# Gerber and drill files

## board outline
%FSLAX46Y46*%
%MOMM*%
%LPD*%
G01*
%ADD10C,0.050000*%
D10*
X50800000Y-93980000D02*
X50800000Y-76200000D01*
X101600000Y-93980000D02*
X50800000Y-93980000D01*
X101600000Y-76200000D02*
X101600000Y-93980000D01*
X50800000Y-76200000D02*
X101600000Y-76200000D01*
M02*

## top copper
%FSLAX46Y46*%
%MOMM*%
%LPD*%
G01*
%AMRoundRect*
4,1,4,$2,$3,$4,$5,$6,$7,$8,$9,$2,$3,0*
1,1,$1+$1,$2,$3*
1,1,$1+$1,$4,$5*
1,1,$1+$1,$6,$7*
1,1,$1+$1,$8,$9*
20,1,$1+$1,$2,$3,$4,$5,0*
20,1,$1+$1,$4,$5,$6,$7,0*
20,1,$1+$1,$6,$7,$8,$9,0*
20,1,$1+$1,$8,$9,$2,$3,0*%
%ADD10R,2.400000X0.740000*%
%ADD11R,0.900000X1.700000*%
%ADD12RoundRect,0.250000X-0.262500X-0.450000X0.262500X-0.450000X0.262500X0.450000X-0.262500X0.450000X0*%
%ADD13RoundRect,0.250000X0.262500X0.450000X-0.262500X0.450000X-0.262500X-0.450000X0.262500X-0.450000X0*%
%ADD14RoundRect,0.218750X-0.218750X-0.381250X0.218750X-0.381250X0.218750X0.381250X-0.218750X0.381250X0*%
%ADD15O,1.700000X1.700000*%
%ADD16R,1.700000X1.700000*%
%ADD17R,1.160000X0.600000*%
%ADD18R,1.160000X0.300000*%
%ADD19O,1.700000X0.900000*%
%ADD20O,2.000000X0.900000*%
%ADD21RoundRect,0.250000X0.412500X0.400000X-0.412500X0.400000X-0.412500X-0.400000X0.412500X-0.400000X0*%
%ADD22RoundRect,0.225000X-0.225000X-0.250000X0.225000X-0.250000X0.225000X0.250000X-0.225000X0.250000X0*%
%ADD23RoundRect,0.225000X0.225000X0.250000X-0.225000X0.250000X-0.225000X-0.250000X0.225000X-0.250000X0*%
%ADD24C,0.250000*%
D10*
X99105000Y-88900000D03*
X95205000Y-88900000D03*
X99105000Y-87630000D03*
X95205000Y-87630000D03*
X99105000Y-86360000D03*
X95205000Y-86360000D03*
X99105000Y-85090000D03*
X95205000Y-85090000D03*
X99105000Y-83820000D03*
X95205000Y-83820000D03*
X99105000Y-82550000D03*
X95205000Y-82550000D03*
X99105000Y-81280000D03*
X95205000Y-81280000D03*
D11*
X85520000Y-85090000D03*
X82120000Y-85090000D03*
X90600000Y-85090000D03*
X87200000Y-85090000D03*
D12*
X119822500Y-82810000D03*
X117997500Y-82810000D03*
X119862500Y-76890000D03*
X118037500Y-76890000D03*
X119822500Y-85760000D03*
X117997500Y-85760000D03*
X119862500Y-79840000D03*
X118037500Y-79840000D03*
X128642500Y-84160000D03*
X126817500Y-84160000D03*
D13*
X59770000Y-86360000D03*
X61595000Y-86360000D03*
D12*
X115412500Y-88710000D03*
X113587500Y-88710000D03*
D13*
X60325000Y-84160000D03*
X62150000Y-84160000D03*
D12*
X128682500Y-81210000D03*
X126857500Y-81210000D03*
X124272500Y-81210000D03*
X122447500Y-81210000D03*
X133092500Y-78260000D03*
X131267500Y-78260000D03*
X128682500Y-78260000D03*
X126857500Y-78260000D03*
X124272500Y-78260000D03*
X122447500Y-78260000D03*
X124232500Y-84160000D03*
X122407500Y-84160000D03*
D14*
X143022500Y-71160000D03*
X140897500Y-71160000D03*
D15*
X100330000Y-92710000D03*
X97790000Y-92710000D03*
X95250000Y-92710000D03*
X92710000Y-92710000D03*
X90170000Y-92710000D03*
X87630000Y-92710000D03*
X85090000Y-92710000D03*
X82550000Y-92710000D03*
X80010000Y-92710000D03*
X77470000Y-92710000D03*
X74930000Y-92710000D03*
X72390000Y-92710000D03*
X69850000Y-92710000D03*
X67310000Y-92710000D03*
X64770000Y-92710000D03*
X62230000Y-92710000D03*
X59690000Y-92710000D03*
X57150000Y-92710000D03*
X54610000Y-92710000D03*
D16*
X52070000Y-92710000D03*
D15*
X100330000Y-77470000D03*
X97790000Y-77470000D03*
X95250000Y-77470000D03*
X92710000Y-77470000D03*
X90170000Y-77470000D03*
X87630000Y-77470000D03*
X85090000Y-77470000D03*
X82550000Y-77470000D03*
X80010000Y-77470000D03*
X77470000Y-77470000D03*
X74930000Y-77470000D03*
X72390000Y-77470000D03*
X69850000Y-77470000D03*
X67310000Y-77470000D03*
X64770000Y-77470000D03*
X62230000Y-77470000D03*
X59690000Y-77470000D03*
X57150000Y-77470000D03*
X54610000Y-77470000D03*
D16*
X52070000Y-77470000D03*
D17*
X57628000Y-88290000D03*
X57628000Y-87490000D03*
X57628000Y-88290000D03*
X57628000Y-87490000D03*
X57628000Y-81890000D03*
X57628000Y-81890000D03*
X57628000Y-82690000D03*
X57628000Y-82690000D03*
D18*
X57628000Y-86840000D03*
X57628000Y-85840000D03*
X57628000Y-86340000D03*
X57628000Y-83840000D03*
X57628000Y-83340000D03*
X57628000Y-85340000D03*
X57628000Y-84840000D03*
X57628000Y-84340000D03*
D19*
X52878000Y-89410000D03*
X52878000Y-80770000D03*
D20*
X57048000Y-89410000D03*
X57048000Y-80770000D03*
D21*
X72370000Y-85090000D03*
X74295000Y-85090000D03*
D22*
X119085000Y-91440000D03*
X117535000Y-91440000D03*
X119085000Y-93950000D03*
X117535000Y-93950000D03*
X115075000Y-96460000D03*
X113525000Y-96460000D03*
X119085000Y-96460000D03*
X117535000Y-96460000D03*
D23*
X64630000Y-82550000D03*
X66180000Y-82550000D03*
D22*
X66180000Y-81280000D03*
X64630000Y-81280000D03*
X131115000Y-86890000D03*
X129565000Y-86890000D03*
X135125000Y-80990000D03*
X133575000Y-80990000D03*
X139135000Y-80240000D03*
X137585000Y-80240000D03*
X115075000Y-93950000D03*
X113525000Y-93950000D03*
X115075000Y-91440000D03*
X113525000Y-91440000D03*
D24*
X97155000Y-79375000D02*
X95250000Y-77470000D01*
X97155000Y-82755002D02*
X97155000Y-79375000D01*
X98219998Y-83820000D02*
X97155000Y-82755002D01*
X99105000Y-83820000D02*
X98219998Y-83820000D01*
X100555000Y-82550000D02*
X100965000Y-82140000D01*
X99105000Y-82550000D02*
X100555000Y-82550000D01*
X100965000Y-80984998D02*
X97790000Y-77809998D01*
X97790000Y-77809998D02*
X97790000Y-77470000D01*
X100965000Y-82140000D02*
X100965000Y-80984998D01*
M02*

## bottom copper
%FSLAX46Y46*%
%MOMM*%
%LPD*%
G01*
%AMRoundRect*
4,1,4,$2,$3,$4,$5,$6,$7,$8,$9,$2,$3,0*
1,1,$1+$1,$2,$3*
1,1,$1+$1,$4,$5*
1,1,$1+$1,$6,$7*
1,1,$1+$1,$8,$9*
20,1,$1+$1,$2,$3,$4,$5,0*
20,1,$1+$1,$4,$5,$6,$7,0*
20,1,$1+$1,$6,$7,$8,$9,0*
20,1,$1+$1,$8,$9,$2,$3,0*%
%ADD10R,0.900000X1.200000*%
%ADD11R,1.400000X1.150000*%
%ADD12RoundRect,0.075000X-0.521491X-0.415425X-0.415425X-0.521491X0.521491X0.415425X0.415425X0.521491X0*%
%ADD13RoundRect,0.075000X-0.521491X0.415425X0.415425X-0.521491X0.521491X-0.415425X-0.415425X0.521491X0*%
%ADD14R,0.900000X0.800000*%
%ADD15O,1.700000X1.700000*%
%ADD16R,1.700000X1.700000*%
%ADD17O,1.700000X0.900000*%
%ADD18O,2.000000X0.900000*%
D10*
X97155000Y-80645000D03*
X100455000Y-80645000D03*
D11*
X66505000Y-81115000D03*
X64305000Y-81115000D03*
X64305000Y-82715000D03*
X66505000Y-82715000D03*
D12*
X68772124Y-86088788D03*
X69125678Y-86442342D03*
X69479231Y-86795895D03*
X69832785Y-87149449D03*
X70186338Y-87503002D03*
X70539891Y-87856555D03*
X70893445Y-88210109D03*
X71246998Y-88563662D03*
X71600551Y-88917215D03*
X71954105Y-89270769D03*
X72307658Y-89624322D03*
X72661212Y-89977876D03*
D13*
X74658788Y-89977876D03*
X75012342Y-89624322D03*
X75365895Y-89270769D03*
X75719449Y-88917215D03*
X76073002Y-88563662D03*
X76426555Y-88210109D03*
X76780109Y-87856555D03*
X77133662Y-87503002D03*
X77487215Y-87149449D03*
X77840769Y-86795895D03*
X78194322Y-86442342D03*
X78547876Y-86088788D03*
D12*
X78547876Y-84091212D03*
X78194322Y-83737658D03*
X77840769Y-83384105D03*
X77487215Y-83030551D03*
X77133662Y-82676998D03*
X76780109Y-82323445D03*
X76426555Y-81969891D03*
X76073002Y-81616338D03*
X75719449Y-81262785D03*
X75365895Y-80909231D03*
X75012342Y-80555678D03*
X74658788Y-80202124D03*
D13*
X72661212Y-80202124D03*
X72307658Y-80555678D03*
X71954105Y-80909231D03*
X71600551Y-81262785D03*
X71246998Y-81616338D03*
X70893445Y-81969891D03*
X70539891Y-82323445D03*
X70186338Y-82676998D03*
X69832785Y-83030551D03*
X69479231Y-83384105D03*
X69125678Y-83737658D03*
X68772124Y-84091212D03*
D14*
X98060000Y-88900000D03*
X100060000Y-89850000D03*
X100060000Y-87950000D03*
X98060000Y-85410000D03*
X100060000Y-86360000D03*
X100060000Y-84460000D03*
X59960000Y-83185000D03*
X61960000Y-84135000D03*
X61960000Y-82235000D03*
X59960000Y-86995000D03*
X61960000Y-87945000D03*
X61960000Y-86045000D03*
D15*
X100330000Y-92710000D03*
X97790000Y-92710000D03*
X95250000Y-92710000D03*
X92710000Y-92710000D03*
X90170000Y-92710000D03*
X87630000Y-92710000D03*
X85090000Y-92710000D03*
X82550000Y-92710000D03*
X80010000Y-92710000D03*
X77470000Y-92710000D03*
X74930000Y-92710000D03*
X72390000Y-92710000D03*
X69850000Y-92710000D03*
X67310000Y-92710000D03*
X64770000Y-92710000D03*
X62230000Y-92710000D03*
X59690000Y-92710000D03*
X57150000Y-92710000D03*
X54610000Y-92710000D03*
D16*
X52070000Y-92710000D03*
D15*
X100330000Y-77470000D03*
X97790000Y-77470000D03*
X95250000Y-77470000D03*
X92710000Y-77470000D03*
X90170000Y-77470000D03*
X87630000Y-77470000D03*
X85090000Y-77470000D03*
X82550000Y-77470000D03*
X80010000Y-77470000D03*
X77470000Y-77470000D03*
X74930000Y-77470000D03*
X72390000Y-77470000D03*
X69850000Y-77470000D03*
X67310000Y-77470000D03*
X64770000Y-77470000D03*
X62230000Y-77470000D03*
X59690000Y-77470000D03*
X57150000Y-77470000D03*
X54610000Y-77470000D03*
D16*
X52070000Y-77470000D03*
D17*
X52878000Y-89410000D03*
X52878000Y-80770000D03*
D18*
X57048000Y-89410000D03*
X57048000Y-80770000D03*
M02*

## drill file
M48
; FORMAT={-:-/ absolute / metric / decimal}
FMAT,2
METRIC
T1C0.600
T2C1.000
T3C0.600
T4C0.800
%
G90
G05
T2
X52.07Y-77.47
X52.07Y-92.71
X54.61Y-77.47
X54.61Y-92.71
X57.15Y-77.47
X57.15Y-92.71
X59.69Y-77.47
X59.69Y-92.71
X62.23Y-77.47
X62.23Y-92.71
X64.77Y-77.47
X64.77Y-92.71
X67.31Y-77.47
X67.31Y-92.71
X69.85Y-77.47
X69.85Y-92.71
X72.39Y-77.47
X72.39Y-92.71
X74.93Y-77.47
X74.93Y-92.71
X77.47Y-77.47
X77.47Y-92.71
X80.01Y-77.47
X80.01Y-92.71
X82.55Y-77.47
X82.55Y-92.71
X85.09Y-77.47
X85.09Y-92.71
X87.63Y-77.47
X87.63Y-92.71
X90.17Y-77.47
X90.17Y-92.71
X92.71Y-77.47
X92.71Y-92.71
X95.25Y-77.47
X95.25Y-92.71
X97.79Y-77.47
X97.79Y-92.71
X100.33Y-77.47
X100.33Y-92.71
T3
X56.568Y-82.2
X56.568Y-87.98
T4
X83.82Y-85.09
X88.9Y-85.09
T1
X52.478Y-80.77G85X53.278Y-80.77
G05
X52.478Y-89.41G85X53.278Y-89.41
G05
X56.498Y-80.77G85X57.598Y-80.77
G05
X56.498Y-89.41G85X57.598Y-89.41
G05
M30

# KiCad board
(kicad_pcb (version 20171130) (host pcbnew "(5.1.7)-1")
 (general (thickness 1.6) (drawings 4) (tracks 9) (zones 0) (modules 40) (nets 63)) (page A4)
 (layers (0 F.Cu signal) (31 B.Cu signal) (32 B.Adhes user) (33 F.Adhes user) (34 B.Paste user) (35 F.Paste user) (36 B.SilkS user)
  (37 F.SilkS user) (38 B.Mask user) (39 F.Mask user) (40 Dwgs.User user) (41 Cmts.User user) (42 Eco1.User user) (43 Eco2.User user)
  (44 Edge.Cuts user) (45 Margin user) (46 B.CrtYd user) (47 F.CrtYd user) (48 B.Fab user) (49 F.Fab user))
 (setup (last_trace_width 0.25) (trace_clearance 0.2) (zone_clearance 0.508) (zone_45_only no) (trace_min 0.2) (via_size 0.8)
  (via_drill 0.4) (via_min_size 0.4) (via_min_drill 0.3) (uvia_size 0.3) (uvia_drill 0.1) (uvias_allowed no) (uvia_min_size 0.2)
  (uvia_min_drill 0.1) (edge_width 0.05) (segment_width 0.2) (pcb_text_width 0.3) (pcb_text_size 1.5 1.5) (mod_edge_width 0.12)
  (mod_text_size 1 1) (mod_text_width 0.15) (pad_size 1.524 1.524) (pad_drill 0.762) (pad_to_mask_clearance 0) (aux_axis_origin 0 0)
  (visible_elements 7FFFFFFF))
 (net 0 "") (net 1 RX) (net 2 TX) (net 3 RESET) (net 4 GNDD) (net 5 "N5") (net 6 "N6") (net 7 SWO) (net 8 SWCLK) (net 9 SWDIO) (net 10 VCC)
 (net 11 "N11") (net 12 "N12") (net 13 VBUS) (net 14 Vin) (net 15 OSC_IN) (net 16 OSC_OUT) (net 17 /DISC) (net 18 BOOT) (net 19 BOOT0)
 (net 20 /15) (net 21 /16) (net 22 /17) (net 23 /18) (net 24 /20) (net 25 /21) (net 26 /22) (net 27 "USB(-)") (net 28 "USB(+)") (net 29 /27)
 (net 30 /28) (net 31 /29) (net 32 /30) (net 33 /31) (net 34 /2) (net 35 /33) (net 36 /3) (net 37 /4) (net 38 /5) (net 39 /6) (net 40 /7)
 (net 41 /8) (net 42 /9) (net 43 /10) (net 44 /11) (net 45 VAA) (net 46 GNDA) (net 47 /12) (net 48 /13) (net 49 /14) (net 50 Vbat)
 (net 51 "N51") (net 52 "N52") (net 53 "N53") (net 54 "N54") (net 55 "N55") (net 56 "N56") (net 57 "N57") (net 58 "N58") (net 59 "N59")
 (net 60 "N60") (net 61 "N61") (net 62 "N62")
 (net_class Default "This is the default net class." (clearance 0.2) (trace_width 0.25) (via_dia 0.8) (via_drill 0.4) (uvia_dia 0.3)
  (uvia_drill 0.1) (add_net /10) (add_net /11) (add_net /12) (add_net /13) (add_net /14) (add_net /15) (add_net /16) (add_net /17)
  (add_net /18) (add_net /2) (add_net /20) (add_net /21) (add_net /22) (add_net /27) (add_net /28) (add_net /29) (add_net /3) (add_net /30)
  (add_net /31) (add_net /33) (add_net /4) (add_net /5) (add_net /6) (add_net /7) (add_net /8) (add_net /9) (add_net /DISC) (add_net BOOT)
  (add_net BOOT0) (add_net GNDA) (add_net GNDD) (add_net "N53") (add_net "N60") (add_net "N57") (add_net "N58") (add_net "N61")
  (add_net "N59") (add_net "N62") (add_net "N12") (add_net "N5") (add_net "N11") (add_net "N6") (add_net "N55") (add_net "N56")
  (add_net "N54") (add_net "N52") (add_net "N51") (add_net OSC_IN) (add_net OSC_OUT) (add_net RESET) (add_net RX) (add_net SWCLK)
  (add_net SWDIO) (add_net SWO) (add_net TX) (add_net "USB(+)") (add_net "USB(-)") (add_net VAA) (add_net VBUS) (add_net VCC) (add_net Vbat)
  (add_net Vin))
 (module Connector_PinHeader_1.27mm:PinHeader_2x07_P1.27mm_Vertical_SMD (layer F.Cu) (at 97.155 85.09)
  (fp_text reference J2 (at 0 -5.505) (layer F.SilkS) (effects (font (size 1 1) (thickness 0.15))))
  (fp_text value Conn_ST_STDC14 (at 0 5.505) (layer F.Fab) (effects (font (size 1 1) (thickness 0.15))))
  (pad 14 smd rect (at 1.95 3.81) (size 2.4 0.74) (layers F.Cu F.Paste F.Mask) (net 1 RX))
  (pad 13 smd rect (at -1.95 3.81) (size 2.4 0.74) (layers F.Cu F.Paste F.Mask) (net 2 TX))
  (pad 12 smd rect (at 1.95 2.54) (size 2.4 0.74) (layers F.Cu F.Paste F.Mask) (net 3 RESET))
  (pad 11 smd rect (at -1.95 2.54) (size 2.4 0.74) (layers F.Cu F.Paste F.Mask) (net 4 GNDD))
  (pad 10 smd rect (at 1.95 1.27) (size 2.4 0.74) (layers F.Cu F.Paste F.Mask) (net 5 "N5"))
  (pad 9 smd rect (at -1.95 1.27) (size 2.4 0.74) (layers F.Cu F.Paste F.Mask) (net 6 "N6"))
  (pad 8 smd rect (at 1.95 0) (size 2.4 0.74) (layers F.Cu F.Paste F.Mask) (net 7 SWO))
  (pad 7 smd rect (at -1.95 0) (size 2.4 0.74) (layers F.Cu F.Paste F.Mask) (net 4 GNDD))
  (pad 6 smd rect (at 1.95 -1.27) (size 2.4 0.74) (layers F.Cu F.Paste F.Mask) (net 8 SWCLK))
  (pad 5 smd rect (at -1.95 -1.27) (size 2.4 0.74) (layers F.Cu F.Paste F.Mask) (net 4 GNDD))
  (pad 4 smd rect (at 1.95 -2.54) (size 2.4 0.74) (layers F.Cu F.Paste F.Mask) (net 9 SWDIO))
  (pad 3 smd rect (at -1.95 -2.54) (size 2.4 0.74) (layers F.Cu F.Paste F.Mask) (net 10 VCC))
  (pad 2 smd rect (at 1.95 -3.81) (size 2.4 0.74) (layers F.Cu F.Paste F.Mask) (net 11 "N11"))
  (pad 1 smd rect (at -1.95 -3.81) (size 2.4 0.74) (layers F.Cu F.Paste F.Mask) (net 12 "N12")))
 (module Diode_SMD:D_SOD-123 (layer B.Cu) (at 98.805 80.645 180)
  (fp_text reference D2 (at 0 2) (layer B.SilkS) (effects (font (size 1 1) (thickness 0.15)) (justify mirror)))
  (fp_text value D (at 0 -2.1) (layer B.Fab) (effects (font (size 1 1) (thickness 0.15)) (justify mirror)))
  (pad 2 smd rect (at 1.65 0 180) (size 0.9 1.2) (layers B.Cu B.Paste B.Mask) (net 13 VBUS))
  (pad 1 smd rect (at -1.65 0 180) (size 0.9 1.2) (layers B.Cu B.Paste B.Mask) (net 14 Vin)))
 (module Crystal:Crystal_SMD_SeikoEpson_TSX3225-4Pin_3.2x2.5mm (layer B.Cu) (at 65.405 81.915 180)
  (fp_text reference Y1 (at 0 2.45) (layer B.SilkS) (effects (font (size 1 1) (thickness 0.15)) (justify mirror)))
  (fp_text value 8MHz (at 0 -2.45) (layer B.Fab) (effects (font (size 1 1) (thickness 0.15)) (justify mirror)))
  (pad 4 smd rect (at -1.1 0.8 180) (size 1.4 1.15) (layers B.Cu B.Paste B.Mask) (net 4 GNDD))
  (pad 3 smd rect (at 1.1 0.8 180) (size 1.4 1.15) (layers B.Cu B.Paste B.Mask) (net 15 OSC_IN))
  (pad 2 smd rect (at 1.1 -0.8 180) (size 1.4 1.15) (layers B.Cu B.Paste B.Mask) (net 4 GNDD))
  (pad 1 smd rect (at -1.1 -0.8 180) (size 1.4 1.15) (layers B.Cu B.Paste B.Mask) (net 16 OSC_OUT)))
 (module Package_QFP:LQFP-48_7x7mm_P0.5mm (layer B.Cu) (at 73.66 85.09 315)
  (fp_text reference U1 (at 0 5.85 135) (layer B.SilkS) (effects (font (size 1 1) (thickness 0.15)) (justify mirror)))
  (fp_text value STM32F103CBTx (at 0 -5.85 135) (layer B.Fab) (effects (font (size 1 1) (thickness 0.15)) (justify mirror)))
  (pad 48 smd roundrect (at -2.75 4.1625 315) (size 0.3 1.475) (layers B.Cu B.Paste B.Mask) (roundrect_rratio 0.25) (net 10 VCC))
  (pad 47 smd roundrect (at -2.25 4.1625 315) (size 0.3 1.475) (layers B.Cu B.Paste B.Mask) (roundrect_rratio 0.25) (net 4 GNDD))
  (pad 46 smd roundrect (at -1.75 4.1625 315) (size 0.3 1.475) (layers B.Cu B.Paste B.Mask) (roundrect_rratio 0.25) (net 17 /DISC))
  (pad 45 smd roundrect (at -1.25 4.1625 315) (size 0.3 1.475) (layers B.Cu B.Paste B.Mask) (roundrect_rratio 0.25) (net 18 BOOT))
  (pad 44 smd roundrect (at -0.75 4.1625 315) (size 0.3 1.475) (layers B.Cu B.Paste B.Mask) (roundrect_rratio 0.25) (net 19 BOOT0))
  (pad 43 smd roundrect (at -0.25 4.1625 315) (size 0.3 1.475) (layers B.Cu B.Paste B.Mask) (roundrect_rratio 0.25) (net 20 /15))
  (pad 42 smd roundrect (at 0.25 4.1625 315) (size 0.3 1.475) (layers B.Cu B.Paste B.Mask) (roundrect_rratio 0.25) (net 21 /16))
  (pad 41 smd roundrect (at 0.75 4.1625 315) (size 0.3 1.475) (layers B.Cu B.Paste B.Mask) (roundrect_rratio 0.25) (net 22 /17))
  (pad 40 smd roundrect (at 1.25 4.1625 315) (size 0.3 1.475) (layers B.Cu B.Paste B.Mask) (roundrect_rratio 0.25) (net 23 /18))
  (pad 39 smd roundrect (at 1.75 4.1625 315) (size 0.3 1.475) (layers B.Cu B.Paste B.Mask) (roundrect_rratio 0.25) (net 7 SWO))
  (pad 38 smd roundrect (at 2.25 4.1625 315) (size 0.3 1.475) (layers B.Cu B.Paste B.Mask) (roundrect_rratio 0.25) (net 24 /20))
  (pad 37 smd roundrect (at 2.75 4.1625 315) (size 0.3 1.475) (layers B.Cu B.Paste B.Mask) (roundrect_rratio 0.25) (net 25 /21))
  (pad 36 smd roundrect (at 4.1625 2.75 315) (size 1.475 0.3) (layers B.Cu B.Paste B.Mask) (roundrect_rratio 0.25) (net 10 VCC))
  (pad 35 smd roundrect (at 4.1625 2.25 315) (size 1.475 0.3) (layers B.Cu B.Paste B.Mask) (roundrect_rratio 0.25) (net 4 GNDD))
  (pad 34 smd roundrect (at 4.1625 1.75 315) (size 1.475 0.3) (layers B.Cu B.Paste B.Mask) (roundrect_rratio 0.25) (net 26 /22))
  (pad 33 smd roundrect (at 4.1625 1.25 315) (size 1.475 0.3) (layers B.Cu B.Paste B.Mask) (roundrect_rratio 0.25) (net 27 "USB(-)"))
  (pad 32 smd roundrect (at 4.1625 0.75 315) (size 1.475 0.3) (layers B.Cu B.Paste B.Mask) (roundrect_rratio 0.25) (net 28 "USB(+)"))
  (pad 31 smd roundrect (at 4.1625 0.25 315) (size 1.475 0.3) (layers B.Cu B.Paste B.Mask) (roundrect_rratio 0.25) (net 1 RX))
  (pad 30 smd roundrect (at 4.1625 -0.25 315) (size 1.475 0.3) (layers B.Cu B.Paste B.Mask) (roundrect_rratio 0.25) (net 2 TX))
  (pad 29 smd roundrect (at 4.1625 -0.75 315) (size 1.475 0.3) (layers B.Cu B.Paste B.Mask) (roundrect_rratio 0.25) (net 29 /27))
  (pad 28 smd roundrect (at 4.1625 -1.25 315) (size 1.475 0.3) (layers B.Cu B.Paste B.Mask) (roundrect_rratio 0.25) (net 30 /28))
  (pad 27 smd roundrect (at 4.1625 -1.75 315) (size 1.475 0.3) (layers B.Cu B.Paste B.Mask) (roundrect_rratio 0.25) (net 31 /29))
  (pad 26 smd roundrect (at 4.1625 -2.25 315) (size 1.475 0.3) (layers B.Cu B.Paste B.Mask) (roundrect_rratio 0.25) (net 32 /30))
  (pad 25 smd roundrect (at 4.1625 -2.75 315) (size 1.475 0.3) (layers B.Cu B.Paste B.Mask) (roundrect_rratio 0.25) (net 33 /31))
  (pad 24 smd roundrect (at 2.75 -4.1625 315) (size 0.3 1.475) (layers B.Cu B.Paste B.Mask) (roundrect_rratio 0.25) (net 10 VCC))
  (pad 23 smd roundrect (at 2.25 -4.1625 315) (size 0.3 1.475) (layers B.Cu B.Paste B.Mask) (roundrect_rratio 0.25) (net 4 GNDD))
  (pad 22 smd roundrect (at 1.75 -4.1625 315) (size 0.3 1.475) (layers B.Cu B.Paste B.Mask) (roundrect_rratio 0.25) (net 9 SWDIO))
  (pad 21 smd roundrect (at 1.25 -4.1625 315) (size 0.3 1.475) (layers B.Cu B.Paste B.Mask) (roundrect_rratio 0.25) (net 8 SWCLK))
  (pad 20 smd roundrect (at 0.75 -4.1625 315) (size 0.3 1.475) (layers B.Cu B.Paste B.Mask) (roundrect_rratio 0.25) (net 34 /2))
  (pad 19 smd roundrect (at 0.25 -4.1625 315) (size 0.3 1.475) (layers B.Cu B.Paste B.Mask) (roundrect_rratio 0.25) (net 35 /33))
  (pad 18 smd roundrect (at -0.25 -4.1625 315) (size 0.3 1.475) (layers B.Cu B.Paste B.Mask) (roundrect_rratio 0.25) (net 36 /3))
  (pad 17 smd roundrect (at -0.75 -4.1625 315) (size 0.3 1.475) (layers B.Cu B.Paste B.Mask) (roundrect_rratio 0.25) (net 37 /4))
  (pad 16 smd roundrect (at -1.25 -4.1625 315) (size 0.3 1.475) (layers B.Cu B.Paste B.Mask) (roundrect_rratio 0.25) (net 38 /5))
  (pad 15 smd roundrect (at -1.75 -4.1625 315) (size 0.3 1.475) (layers B.Cu B.Paste B.Mask) (roundrect_rratio 0.25) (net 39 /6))
  (pad 14 smd roundrect (at -2.25 -4.1625 315) (size 0.3 1.475) (layers B.Cu B.Paste B.Mask) (roundrect_rratio 0.25) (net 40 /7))
  (pad 13 smd roundrect (at -2.75 -4.1625 315) (size 0.3 1.475) (layers B.Cu B.Paste B.Mask) (roundrect_rratio 0.25) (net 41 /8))
  (pad 12 smd roundrect (at -4.1625 -2.75 315) (size 1.475 0.3) (layers B.Cu B.Paste B.Mask) (roundrect_rratio 0.25) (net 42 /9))
  (pad 11 smd roundrect (at -4.1625 -2.25 315) (size 1.475 0.3) (layers B.Cu B.Paste B.Mask) (roundrect_rratio 0.25) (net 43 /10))
  (pad 10 smd roundrect (at -4.1625 -1.75 315) (size 1.475 0.3) (layers B.Cu B.Paste B.Mask) (roundrect_rratio 0.25) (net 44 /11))
  (pad 9 smd roundrect (at -4.1625 -1.25 315) (size 1.475 0.3) (layers B.Cu B.Paste B.Mask) (roundrect_rratio 0.25) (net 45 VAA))
  (pad 8 smd roundrect (at -4.1625 -0.75 315) (size 1.475 0.3) (layers B.Cu B.Paste B.Mask) (roundrect_rratio 0.25) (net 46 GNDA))
  (pad 7 smd roundrect (at -4.1625 -0.25 315) (size 1.475 0.3) (layers B.Cu B.Paste B.Mask) (roundrect_rratio 0.25) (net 3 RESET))
  (pad 6 smd roundrect (at -4.1625 0.25 315) (size 1.475 0.3) (layers B.Cu B.Paste B.Mask) (roundrect_rratio 0.25) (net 16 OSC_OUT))
  (pad 5 smd roundrect (at -4.1625 0.75 315) (size 1.475 0.3) (layers B.Cu B.Paste B.Mask) (roundrect_rratio 0.25) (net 15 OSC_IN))
  (pad 4 smd roundrect (at -4.1625 1.25 315) (size 1.475 0.3) (layers B.Cu B.Paste B.Mask) (roundrect_rratio 0.25) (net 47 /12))
  (pad 3 smd roundrect (at -4.1625 1.75 315) (size 1.475 0.3) (layers B.Cu B.Paste B.Mask) (roundrect_rratio 0.25) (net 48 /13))
  (pad 2 smd roundrect (at -4.1625 2.25 315) (size 1.475 0.3) (layers B.Cu B.Paste B.Mask) (roundrect_rratio 0.25) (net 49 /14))
  (pad 1 smd roundrect (at -4.1625 2.75 315) (size 1.475 0.3) (layers B.Cu B.Paste B.Mask) (roundrect_rratio 0.25) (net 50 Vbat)))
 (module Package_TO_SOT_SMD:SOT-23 (layer B.Cu) (at 99.06 88.9 180)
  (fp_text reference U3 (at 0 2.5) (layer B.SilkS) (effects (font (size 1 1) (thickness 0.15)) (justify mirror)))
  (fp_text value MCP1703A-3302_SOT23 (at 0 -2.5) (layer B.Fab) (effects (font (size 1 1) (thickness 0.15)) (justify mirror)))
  (pad 3 smd rect (at 1 0 180) (size 0.9 0.8) (layers B.Cu B.Paste B.Mask) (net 14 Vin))
  (pad 2 smd rect (at -1 -0.95 180) (size 0.9 0.8) (layers B.Cu B.Paste B.Mask) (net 45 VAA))
  (pad 1 smd rect (at -1 0.95 180) (size 0.9 0.8) (layers B.Cu B.Paste B.Mask) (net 4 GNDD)))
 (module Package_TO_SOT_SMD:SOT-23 (layer B.Cu) (at 99.06 85.41 180)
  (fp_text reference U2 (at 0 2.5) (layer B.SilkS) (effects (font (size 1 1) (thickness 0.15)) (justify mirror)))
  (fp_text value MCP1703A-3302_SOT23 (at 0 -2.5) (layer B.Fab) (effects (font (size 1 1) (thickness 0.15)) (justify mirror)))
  (pad 3 smd rect (at 1 0 180) (size 0.9 0.8) (layers B.Cu B.Paste B.Mask) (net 14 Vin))
  (pad 2 smd rect (at -1 -0.95 180) (size 0.9 0.8) (layers B.Cu B.Paste B.Mask) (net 10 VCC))
  (pad 1 smd rect (at -1 0.95 180) (size 0.9 0.8) (layers B.Cu B.Paste B.Mask) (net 4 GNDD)))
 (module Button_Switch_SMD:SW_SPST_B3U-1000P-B (layer F.Cu) (at 83.82 85.09)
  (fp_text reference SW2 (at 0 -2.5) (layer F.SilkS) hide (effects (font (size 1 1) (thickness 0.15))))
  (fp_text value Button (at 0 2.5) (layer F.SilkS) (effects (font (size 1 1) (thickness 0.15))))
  (pad "" np_thru_hole circle (at 0 0) (size 0.8 0.8) (drill 0.8) (layers *.Cu *.Mask))
  (pad 2 smd rect (at 1.7 0) (size 0.9 1.7) (layers F.Cu F.Paste F.Mask) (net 19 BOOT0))
  (pad 1 smd rect (at -1.7 0) (size 0.9 1.7) (layers F.Cu F.Paste F.Mask) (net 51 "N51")))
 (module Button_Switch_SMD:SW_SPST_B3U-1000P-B (layer F.Cu) (at 88.9 85.09)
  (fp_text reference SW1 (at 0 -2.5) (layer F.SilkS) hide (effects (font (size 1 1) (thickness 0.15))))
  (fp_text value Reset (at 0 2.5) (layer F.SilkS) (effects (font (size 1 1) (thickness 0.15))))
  (pad "" np_thru_hole circle (at 0 0) (size 0.8 0.8) (drill 0.8) (layers *.Cu *.Mask))
  (pad 2 smd rect (at 1.7 0) (size 0.9 1.7) (layers F.Cu F.Paste F.Mask) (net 3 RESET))
  (pad 1 smd rect (at -1.7 0) (size 0.9 1.7) (layers F.Cu F.Paste F.Mask) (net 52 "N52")))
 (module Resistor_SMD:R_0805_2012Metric (layer F.Cu) (at 118.91 82.81)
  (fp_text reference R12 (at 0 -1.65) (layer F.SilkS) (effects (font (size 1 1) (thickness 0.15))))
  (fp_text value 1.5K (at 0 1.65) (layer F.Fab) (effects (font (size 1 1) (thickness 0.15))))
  (pad 2 smd roundrect (at 0.9125 0) (size 1.025 1.4) (layers F.Cu F.Paste F.Mask) (roundrect_rratio 0.243902) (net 35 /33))
  (pad 1 smd roundrect (at -0.9125 0) (size 1.025 1.4) (layers F.Cu F.Paste F.Mask) (roundrect_rratio 0.243902) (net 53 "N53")))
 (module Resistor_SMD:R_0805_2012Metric (layer F.Cu) (at 118.95 76.89)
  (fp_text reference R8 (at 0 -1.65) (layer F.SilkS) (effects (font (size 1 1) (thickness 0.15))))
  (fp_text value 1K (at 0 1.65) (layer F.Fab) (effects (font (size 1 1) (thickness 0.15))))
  (pad 2 smd roundrect (at 0.9125 0) (size 1.025 1.4) (layers F.Cu F.Paste F.Mask) (roundrect_rratio 0.243902) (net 17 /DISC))
  (pad 1 smd roundrect (at -0.9125 0) (size 1.025 1.4) (layers F.Cu F.Paste F.Mask) (roundrect_rratio 0.243902) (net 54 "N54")))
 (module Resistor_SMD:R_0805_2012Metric (layer F.Cu) (at 118.91 85.76)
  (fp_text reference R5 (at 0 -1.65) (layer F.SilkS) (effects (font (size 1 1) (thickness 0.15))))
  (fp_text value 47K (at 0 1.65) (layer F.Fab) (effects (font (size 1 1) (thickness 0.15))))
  (pad 2 smd roundrect (at 0.9125 0) (size 1.025 1.4) (layers F.Cu F.Paste F.Mask) (roundrect_rratio 0.243902) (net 54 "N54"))
  (pad 1 smd roundrect (at -0.9125 0) (size 1.025 1.4) (layers F.Cu F.Paste F.Mask) (roundrect_rratio 0.243902) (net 10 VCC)))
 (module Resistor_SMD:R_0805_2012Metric (layer F.Cu) (at 118.95 79.84)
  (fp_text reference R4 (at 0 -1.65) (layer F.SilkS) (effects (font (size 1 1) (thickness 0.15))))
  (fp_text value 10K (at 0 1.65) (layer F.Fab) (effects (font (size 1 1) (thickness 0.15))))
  (pad 2 smd roundrect (at 0.9125 0) (size 1.025 1.4) (layers F.Cu F.Paste F.Mask) (roundrect_rratio 0.243902) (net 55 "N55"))
  (pad 1 smd roundrect (at -0.9125 0) (size 1.025 1.4) (layers F.Cu F.Paste F.Mask) (roundrect_rratio 0.243902) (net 13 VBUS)))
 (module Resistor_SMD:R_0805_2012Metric (layer F.Cu) (at 127.73 84.16)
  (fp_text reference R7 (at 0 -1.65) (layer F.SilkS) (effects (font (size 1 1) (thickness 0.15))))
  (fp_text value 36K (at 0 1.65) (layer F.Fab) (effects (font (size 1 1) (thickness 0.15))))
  (pad 2 smd roundrect (at 0.9125 0) (size 1.025 1.4) (layers F.Cu F.Paste F.Mask) (roundrect_rratio 0.243902) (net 4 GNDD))
  (pad 1 smd roundrect (at -0.9125 0) (size 1.025 1.4) (layers F.Cu F.Paste F.Mask) (roundrect_rratio 0.243902) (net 55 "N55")))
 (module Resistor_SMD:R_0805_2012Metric (layer F.Cu) (at 60.6825 86.36 180)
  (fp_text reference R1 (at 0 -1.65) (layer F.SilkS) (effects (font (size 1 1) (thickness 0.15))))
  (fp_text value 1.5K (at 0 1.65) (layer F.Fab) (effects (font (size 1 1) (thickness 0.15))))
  (pad 2 smd roundrect (at 0.9125 0 180) (size 1.025 1.4) (layers F.Cu F.Paste F.Mask) (roundrect_rratio 0.243902) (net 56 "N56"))
  (pad 1 smd roundrect (at -0.9125 0 180) (size 1.025 1.4) (layers F.Cu F.Paste F.Mask) (roundrect_rratio 0.243902) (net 28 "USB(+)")))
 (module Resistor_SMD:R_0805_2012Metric (layer F.Cu) (at 114.5 88.71)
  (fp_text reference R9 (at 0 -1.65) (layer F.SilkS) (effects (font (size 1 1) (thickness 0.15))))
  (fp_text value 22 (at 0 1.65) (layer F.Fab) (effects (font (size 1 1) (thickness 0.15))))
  (pad 2 smd roundrect (at 0.9125 0) (size 1.025 1.4) (layers F.Cu F.Paste F.Mask) (roundrect_rratio 0.243902) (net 28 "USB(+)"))
  (pad 1 smd roundrect (at -0.9125 0) (size 1.025 1.4) (layers F.Cu F.Paste F.Mask) (roundrect_rratio 0.243902) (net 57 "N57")))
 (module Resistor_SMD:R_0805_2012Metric (layer F.Cu) (at 61.2375 84.16 180)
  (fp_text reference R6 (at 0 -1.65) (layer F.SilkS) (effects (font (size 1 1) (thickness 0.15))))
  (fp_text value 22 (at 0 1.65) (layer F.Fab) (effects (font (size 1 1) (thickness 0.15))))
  (pad 2 smd roundrect (at 0.9125 0 180) (size 1.025 1.4) (layers F.Cu F.Paste F.Mask) (roundrect_rratio 0.243902) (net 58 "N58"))
  (pad 1 smd roundrect (at -0.9125 0 180) (size 1.025 1.4) (layers F.Cu F.Paste F.Mask) (roundrect_rratio 0.243902) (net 27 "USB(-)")))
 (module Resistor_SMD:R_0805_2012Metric (layer F.Cu) (at 127.77 81.21)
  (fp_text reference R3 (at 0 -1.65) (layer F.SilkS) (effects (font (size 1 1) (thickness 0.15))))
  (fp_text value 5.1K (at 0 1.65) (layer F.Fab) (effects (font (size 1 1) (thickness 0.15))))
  (pad 2 smd roundrect (at 0.9125 0) (size 1.025 1.4) (layers F.Cu F.Paste F.Mask) (roundrect_rratio 0.243902) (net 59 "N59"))
  (pad 1 smd roundrect (at -0.9125 0) (size 1.025 1.4) (layers F.Cu F.Paste F.Mask) (roundrect_rratio 0.243902) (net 4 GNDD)))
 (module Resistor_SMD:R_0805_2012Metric (layer F.Cu) (at 123.36 81.21)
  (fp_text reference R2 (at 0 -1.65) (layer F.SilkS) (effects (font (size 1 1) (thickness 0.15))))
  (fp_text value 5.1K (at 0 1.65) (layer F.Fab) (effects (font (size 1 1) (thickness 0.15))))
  (pad 2 smd roundrect (at 0.9125 0) (size 1.025 1.4) (layers F.Cu F.Paste F.Mask) (roundrect_rratio 0.243902) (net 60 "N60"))
  (pad 1 smd roundrect (at -0.9125 0) (size 1.025 1.4) (layers F.Cu F.Paste F.Mask) (roundrect_rratio 0.243902) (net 4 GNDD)))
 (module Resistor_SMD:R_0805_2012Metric (layer F.Cu) (at 132.18 78.26)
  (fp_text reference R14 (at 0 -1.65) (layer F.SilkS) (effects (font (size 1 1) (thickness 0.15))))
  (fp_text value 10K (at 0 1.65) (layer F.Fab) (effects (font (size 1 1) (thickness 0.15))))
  (pad 2 smd roundrect (at 0.9125 0) (size 1.025 1.4) (layers F.Cu F.Paste F.Mask) (roundrect_rratio 0.243902) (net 4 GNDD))
  (pad 1 smd roundrect (at -0.9125 0) (size 1.025 1.4) (layers F.Cu F.Paste F.Mask) (roundrect_rratio 0.243902) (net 51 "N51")))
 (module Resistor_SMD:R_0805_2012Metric (layer F.Cu) (at 127.77 78.26)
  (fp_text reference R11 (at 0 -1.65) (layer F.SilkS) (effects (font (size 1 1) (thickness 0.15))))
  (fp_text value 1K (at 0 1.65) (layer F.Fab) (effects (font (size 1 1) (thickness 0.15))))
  (pad 2 smd roundrect (at 0.9125 0) (size 1.025 1.4) (layers F.Cu F.Paste F.Mask) (roundrect_rratio 0.243902) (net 19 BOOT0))
  (pad 1 smd roundrect (at -0.9125 0) (size 1.025 1.4) (layers F.Cu F.Paste F.Mask) (roundrect_rratio 0.243902) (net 10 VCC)))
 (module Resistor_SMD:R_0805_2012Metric (layer F.Cu) (at 123.36 78.26)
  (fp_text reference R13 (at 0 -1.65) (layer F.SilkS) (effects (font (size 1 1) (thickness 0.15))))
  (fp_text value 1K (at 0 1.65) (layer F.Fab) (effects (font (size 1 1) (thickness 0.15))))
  (pad 2 smd roundrect (at 0.9125 0) (size 1.025 1.4) (layers F.Cu F.Paste F.Mask) (roundrect_rratio 0.243902) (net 4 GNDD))
  (pad 1 smd roundrect (at -0.9125 0) (size 1.025 1.4) (layers F.Cu F.Paste F.Mask) (roundrect_rratio 0.243902) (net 52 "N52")))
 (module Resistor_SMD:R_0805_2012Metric (layer F.Cu) (at 123.32 84.16)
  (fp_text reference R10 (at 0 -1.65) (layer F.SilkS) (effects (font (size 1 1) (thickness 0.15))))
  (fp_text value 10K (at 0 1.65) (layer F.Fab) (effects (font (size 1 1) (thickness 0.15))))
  (pad 2 smd roundrect (at 0.9125 0) (size 1.025 1.4) (layers F.Cu F.Paste F.Mask) (roundrect_rratio 0.243902) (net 3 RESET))
  (pad 1 smd roundrect (at -0.9125 0) (size 1.025 1.4) (layers F.Cu F.Paste F.Mask) (roundrect_rratio 0.243902) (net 10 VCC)))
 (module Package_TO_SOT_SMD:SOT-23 (layer B.Cu) (at 60.96 83.185 180)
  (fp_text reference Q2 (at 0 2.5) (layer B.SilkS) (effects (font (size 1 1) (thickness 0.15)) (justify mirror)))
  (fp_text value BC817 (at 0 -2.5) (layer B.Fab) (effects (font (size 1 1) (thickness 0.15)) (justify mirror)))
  (pad 3 smd rect (at 1 0 180) (size 0.9 0.8) (layers B.Cu B.Paste B.Mask) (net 55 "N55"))
  (pad 2 smd rect (at -1 -0.95 180) (size 0.9 0.8) (layers B.Cu B.Paste B.Mask) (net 4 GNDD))
  (pad 1 smd rect (at -1 0.95 180) (size 0.9 0.8) (layers B.Cu B.Paste B.Mask) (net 54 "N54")))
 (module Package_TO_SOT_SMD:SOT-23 (layer B.Cu) (at 60.96 86.995 180)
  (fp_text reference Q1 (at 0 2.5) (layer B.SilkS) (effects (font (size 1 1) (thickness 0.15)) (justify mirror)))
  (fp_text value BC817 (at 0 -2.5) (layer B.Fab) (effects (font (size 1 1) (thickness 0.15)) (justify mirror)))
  (pad 3 smd rect (at 1 0 180) (size 0.9 0.8) (layers B.Cu B.Paste B.Mask) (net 10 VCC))
  (pad 2 smd rect (at -1 -0.95 180) (size 0.9 0.8) (layers B.Cu B.Paste B.Mask) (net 56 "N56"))
  (pad 1 smd rect (at -1 0.95 180) (size 0.9 0.8) (layers B.Cu B.Paste B.Mask) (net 55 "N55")))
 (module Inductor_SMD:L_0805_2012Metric (layer F.Cu) (at 141.96 71.16)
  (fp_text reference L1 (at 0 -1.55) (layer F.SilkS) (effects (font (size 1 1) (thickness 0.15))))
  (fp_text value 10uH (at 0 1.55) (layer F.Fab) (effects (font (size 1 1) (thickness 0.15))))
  (pad 2 smd roundrect (at 1.0625 0) (size 0.875 1.2) (layers F.Cu F.Paste F.Mask) (roundrect_rratio 0.25) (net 4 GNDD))
  (pad 1 smd roundrect (at -1.0625 0) (size 0.875 1.2) (layers F.Cu F.Paste F.Mask) (roundrect_rratio 0.25) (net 46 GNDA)))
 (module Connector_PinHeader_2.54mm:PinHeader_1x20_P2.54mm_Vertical (layer B.Cu) (at 52.07 92.71 270)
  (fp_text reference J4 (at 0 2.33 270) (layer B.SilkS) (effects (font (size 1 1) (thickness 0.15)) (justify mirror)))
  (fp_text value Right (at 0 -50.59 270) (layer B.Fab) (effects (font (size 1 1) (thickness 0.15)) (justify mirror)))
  (pad 20 thru_hole oval (at 0 -48.26 270) (size 1.7 1.7) (drill 1) (layers *.Cu *.Mask) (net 33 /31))
  (pad 19 thru_hole oval (at 0 -45.72 270) (size 1.7 1.7) (drill 1) (layers *.Cu *.Mask) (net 32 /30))
  (pad 18 thru_hole oval (at 0 -43.18 270) (size 1.7 1.7) (drill 1) (layers *.Cu *.Mask) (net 31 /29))
  (pad 17 thru_hole oval (at 0 -40.64 270) (size 1.7 1.7) (drill 1) (layers *.Cu *.Mask) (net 30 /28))
  (pad 16 thru_hole oval (at 0 -38.1 270) (size 1.7 1.7) (drill 1) (layers *.Cu *.Mask) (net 29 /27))
  (pad 15 thru_hole oval (at 0 -35.56 270) (size 1.7 1.7) (drill 1) (layers *.Cu *.Mask) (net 2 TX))
  (pad 14 thru_hole oval (at 0 -33.02 270) (size 1.7 1.7) (drill 1) (layers *.Cu *.Mask) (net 1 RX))
  (pad 13 thru_hole oval (at 0 -30.48 270) (size 1.7 1.7) (drill 1) (layers *.Cu *.Mask) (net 28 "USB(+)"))
  (pad 12 thru_hole oval (at 0 -27.94 270) (size 1.7 1.7) (drill 1) (layers *.Cu *.Mask) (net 27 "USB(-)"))
  (pad 11 thru_hole oval (at 0 -25.4 270) (size 1.7 1.7) (drill 1) (layers *.Cu *.Mask) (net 26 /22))
  (pad 10 thru_hole oval (at 0 -22.86 270) (size 1.7 1.7) (drill 1) (layers *.Cu *.Mask) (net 25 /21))
  (pad 9 thru_hole oval (at 0 -20.32 270) (size 1.7 1.7) (drill 1) (layers *.Cu *.Mask) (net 24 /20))
  (pad 8 thru_hole oval (at 0 -17.78 270) (size 1.7 1.7) (drill 1) (layers *.Cu *.Mask) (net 7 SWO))
  (pad 7 thru_hole oval (at 0 -15.24 270) (size 1.7 1.7) (drill 1) (layers *.Cu *.Mask) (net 23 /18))
  (pad 6 thru_hole oval (at 0 -12.7 270) (size 1.7 1.7) (drill 1) (layers *.Cu *.Mask) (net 22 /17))
  (pad 5 thru_hole oval (at 0 -10.16 270) (size 1.7 1.7) (drill 1) (layers *.Cu *.Mask) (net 21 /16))
  (pad 4 thru_hole oval (at 0 -7.62 270) (size 1.7 1.7) (drill 1) (layers *.Cu *.Mask) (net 20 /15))
  (pad 3 thru_hole oval (at 0 -5.08 270) (size 1.7 1.7) (drill 1) (layers *.Cu *.Mask) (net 18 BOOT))
  (pad 2 thru_hole oval (at 0 -2.54 270) (size 1.7 1.7) (drill 1) (layers *.Cu *.Mask) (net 4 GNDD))
  (pad 1 thru_hole rect (at 0 0 270) (size 1.7 1.7) (drill 1) (layers *.Cu *.Mask) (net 10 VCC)))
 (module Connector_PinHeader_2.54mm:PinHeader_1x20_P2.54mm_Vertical (layer B.Cu) (at 52.07 77.47 270)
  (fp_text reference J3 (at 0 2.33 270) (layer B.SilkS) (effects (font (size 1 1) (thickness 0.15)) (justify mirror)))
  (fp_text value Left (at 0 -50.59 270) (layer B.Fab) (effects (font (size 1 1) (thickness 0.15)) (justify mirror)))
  (pad 20 thru_hole oval (at 0 -48.26 270) (size 1.7 1.7) (drill 1) (layers *.Cu *.Mask) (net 14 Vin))
  (pad 19 thru_hole oval (at 0 -45.72 270) (size 1.7 1.7) (drill 1) (layers *.Cu *.Mask) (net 9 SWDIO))
  (pad 18 thru_hole oval (at 0 -43.18 270) (size 1.7 1.7) (drill 1) (layers *.Cu *.Mask) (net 8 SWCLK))
  (pad 17 thru_hole oval (at 0 -40.64 270) (size 1.7 1.7) (drill 1) (layers *.Cu *.Mask) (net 34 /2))
  (pad 16 thru_hole oval (at 0 -38.1 270) (size 1.7 1.7) (drill 1) (layers *.Cu *.Mask) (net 36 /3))
  (pad 15 thru_hole oval (at 0 -35.56 270) (size 1.7 1.7) (drill 1) (layers *.Cu *.Mask) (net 37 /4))
  (pad 14 thru_hole oval (at 0 -33.02 270) (size 1.7 1.7) (drill 1) (layers *.Cu *.Mask) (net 38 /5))
  (pad 13 thru_hole oval (at 0 -30.48 270) (size 1.7 1.7) (drill 1) (layers *.Cu *.Mask) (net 39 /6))
  (pad 12 thru_hole oval (at 0 -27.94 270) (size 1.7 1.7) (drill 1) (layers *.Cu *.Mask) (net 40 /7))
  (pad 11 thru_hole oval (at 0 -25.4 270) (size 1.7 1.7) (drill 1) (layers *.Cu *.Mask) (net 41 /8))
  (pad 10 thru_hole oval (at 0 -22.86 270) (size 1.7 1.7) (drill 1) (layers *.Cu *.Mask) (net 42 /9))
  (pad 9 thru_hole oval (at 0 -20.32 270) (size 1.7 1.7) (drill 1) (layers *.Cu *.Mask) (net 43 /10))
  (pad 8 thru_hole oval (at 0 -17.78 270) (size 1.7 1.7) (drill 1) (layers *.Cu *.Mask) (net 44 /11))
  (pad 7 thru_hole oval (at 0 -15.24 270) (size 1.7 1.7) (drill 1) (layers *.Cu *.Mask) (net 3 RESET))
  (pad 6 thru_hole oval (at 0 -12.7 270) (size 1.7 1.7) (drill 1) (layers *.Cu *.Mask) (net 47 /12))
  (pad 5 thru_hole oval (at 0 -10.16 270) (size 1.7 1.7) (drill 1) (layers *.Cu *.Mask) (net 49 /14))
  (pad 4 thru_hole oval (at 0 -7.62 270) (size 1.7 1.7) (drill 1) (layers *.Cu *.Mask) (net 48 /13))
  (pad 3 thru_hole oval (at 0 -5.08 270) (size 1.7 1.7) (drill 1) (layers *.Cu *.Mask) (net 50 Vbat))
  (pad 2 thru_hole oval (at 0 -2.54 270) (size 1.7 1.7) (drill 1) (layers *.Cu *.Mask) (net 46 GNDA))
  (pad 1 thru_hole rect (at 0 0 270) (size 1.7 1.7) (drill 1) (layers *.Cu *.Mask) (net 45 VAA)))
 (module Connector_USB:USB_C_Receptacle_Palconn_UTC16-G (layer F.Cu) (at 55.118 85.09 270)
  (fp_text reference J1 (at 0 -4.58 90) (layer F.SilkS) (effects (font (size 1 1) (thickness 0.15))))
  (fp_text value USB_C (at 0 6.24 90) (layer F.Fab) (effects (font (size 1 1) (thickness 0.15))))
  (pad A12 smd rect (at 3.2 -2.51 270) (size 0.6 1.16) (layers F.Cu F.Paste F.Mask) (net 4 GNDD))
  (pad A9 smd rect (at 2.4 -2.51 270) (size 0.6 1.16) (layers F.Cu F.Paste F.Mask) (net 13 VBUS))
  (pad B1 smd rect (at 3.2 -2.51 270) (size 0.6 1.16) (layers F.Cu F.Paste F.Mask) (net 4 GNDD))
  (pad B4 smd rect (at 2.4 -2.51 270) (size 0.6 1.16) (layers F.Cu F.Paste F.Mask) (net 13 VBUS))
  (pad B12 smd rect (at -3.2 -2.51 270) (size 0.6 1.16) (layers F.Cu F.Paste F.Mask) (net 4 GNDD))
  (pad A1 smd rect (at -3.2 -2.51 270) (size 0.6 1.16) (layers F.Cu F.Paste F.Mask) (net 4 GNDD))
  (pad B9 smd rect (at -2.4 -2.51 270) (size 0.6 1.16) (layers F.Cu F.Paste F.Mask) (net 13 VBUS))
  (pad A4 smd rect (at -2.4 -2.51 270) (size 0.6 1.16) (layers F.Cu F.Paste F.Mask) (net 13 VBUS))
  (pad "" np_thru_hole circle (at -2.89 -1.45 90) (size 0.6 0.6) (drill 0.6) (layers *.Cu *.Mask))
  (pad "" np_thru_hole circle (at 2.89 -1.45 90) (size 0.6 0.6) (drill 0.6) (layers *.Cu *.Mask))
  (pad B5 smd rect (at 1.75 -2.51 90) (size 0.3 1.16) (layers F.Cu F.Paste F.Mask) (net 59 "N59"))
  (pad B6 smd rect (at 0.75 -2.51 90) (size 0.3 1.16) (layers F.Cu F.Paste F.Mask) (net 57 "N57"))
  (pad A8 smd rect (at 1.25 -2.51 90) (size 0.3 1.16) (layers F.Cu F.Paste F.Mask) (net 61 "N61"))
  (pad A5 smd rect (at -1.25 -2.51 90) (size 0.3 1.16) (layers F.Cu F.Paste F.Mask) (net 60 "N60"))
  (pad B8 smd rect (at -1.75 -2.51 90) (size 0.3 1.16) (layers F.Cu F.Paste F.Mask) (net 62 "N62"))
  (pad A7 smd rect (at 0.25 -2.51 90) (size 0.3 1.16) (layers F.Cu F.Paste F.Mask) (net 58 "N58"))
  (pad A6 smd rect (at -0.25 -2.51 90) (size 0.3 1.16) (layers F.Cu F.Paste F.Mask) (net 57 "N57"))
  (pad B7 smd rect (at -0.75 -2.51 90) (size 0.3 1.16) (layers F.Cu F.Paste F.Mask) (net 58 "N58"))
  (pad S1 thru_hole oval (at 4.32 2.24) (size 1.7 0.9) (drill oval 1.4 0.6) (layers *.Cu *.Mask) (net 4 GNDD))
  (pad S1 thru_hole oval (at -4.32 2.24) (size 1.7 0.9) (drill oval 1.4 0.6) (layers *.Cu *.Mask) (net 4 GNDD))
  (pad S1 thru_hole oval (at 4.32 -1.93) (size 2 0.9) (drill oval 1.7 0.6) (layers *.Cu *.Mask) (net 4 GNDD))
  (pad S1 thru_hole oval (at -4.32 -1.93) (size 2 0.9) (drill oval 1.7 0.6) (layers *.Cu *.Mask) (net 4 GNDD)))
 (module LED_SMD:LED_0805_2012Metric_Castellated (layer F.Cu) (at 73.3325 85.09 180)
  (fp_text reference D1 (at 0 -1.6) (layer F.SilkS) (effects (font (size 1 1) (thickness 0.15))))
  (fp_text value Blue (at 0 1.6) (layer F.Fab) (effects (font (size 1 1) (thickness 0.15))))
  (pad 2 smd roundrect (at 0.9625 0 180) (size 1.325 1.3) (layers F.Cu F.Paste F.Mask) (roundrect_rratio 0.192308) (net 53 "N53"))
  (pad 1 smd roundrect (at -0.9625 0 180) (size 1.325 1.3) (layers F.Cu F.Paste F.Mask) (roundrect_rratio 0.192308) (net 4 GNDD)))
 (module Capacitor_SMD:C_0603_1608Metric (layer F.Cu) (at 118.31 91.44)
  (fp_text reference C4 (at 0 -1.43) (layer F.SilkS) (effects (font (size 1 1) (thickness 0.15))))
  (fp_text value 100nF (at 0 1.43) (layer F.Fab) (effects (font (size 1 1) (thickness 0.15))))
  (pad 2 smd roundrect (at 0.775 0) (size 0.9 0.95) (layers F.Cu F.Paste F.Mask) (roundrect_rratio 0.25) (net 4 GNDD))
  (pad 1 smd roundrect (at -0.775 0) (size 0.9 0.95) (layers F.Cu F.Paste F.Mask) (roundrect_rratio 0.25) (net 10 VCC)))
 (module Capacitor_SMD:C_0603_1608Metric (layer F.Cu) (at 118.31 93.95)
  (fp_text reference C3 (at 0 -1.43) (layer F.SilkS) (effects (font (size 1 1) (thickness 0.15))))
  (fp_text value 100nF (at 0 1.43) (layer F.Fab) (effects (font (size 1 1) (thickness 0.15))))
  (pad 2 smd roundrect (at 0.775 0) (size 0.9 0.95) (layers F.Cu F.Paste F.Mask) (roundrect_rratio 0.25) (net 4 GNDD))
  (pad 1 smd roundrect (at -0.775 0) (size 0.9 0.95) (layers F.Cu F.Paste F.Mask) (roundrect_rratio 0.25) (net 10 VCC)))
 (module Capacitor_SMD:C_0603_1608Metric (layer F.Cu) (at 114.3 96.46)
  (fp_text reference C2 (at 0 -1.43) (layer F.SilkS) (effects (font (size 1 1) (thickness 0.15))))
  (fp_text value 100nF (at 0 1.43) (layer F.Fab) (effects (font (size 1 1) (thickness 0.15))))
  (pad 2 smd roundrect (at 0.775 0) (size 0.9 0.95) (layers F.Cu F.Paste F.Mask) (roundrect_rratio 0.25) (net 4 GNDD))
  (pad 1 smd roundrect (at -0.775 0) (size 0.9 0.95) (layers F.Cu F.Paste F.Mask) (roundrect_rratio 0.25) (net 10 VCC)))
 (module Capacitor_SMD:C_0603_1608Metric (layer F.Cu) (at 118.31 96.46)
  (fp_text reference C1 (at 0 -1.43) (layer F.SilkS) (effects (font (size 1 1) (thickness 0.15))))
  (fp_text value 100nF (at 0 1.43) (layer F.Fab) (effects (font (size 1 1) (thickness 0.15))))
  (pad 2 smd roundrect (at 0.775 0) (size 0.9 0.95) (layers F.Cu F.Paste F.Mask) (roundrect_rratio 0.25) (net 46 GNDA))
  (pad 1 smd roundrect (at -0.775 0) (size 0.9 0.95) (layers F.Cu F.Paste F.Mask) (roundrect_rratio 0.25) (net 45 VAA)))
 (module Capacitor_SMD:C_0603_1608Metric (layer F.Cu) (at 65.405 82.55 180)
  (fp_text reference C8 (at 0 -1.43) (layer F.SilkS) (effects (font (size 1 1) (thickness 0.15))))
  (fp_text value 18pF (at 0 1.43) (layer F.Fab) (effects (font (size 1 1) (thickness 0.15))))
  (pad 2 smd roundrect (at 0.775 0 180) (size 0.9 0.95) (layers F.Cu F.Paste F.Mask) (roundrect_rratio 0.25) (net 4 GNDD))
  (pad 1 smd roundrect (at -0.775 0 180) (size 0.9 0.95) (layers F.Cu F.Paste F.Mask) (roundrect_rratio 0.25) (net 15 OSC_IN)))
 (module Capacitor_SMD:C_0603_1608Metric (layer F.Cu) (at 65.405 81.28)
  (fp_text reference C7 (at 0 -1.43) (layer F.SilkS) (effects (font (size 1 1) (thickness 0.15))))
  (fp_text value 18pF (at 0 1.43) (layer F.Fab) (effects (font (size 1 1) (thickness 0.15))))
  (pad 2 smd roundrect (at 0.775 0) (size 0.9 0.95) (layers F.Cu F.Paste F.Mask) (roundrect_rratio 0.25) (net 4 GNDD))
  (pad 1 smd roundrect (at -0.775 0) (size 0.9 0.95) (layers F.Cu F.Paste F.Mask) (roundrect_rratio 0.25) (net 16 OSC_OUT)))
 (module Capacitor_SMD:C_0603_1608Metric (layer F.Cu) (at 130.34 86.89)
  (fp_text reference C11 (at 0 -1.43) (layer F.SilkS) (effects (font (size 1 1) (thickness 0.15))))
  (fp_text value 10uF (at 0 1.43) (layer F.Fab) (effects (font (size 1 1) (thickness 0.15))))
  (pad 2 smd roundrect (at 0.775 0) (size 0.9 0.95) (layers F.Cu F.Paste F.Mask) (roundrect_rratio 0.25) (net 46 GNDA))
  (pad 1 smd roundrect (at -0.775 0) (size 0.9 0.95) (layers F.Cu F.Paste F.Mask) (roundrect_rratio 0.25) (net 45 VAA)))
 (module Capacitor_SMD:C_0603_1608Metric (layer F.Cu) (at 134.35 80.99)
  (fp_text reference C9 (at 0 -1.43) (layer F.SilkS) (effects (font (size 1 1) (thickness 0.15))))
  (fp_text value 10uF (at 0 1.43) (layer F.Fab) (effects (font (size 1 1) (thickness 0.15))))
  (pad 2 smd roundrect (at 0.775 0) (size 0.9 0.95) (layers F.Cu F.Paste F.Mask) (roundrect_rratio 0.25) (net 4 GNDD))
  (pad 1 smd roundrect (at -0.775 0) (size 0.9 0.95) (layers F.Cu F.Paste F.Mask) (roundrect_rratio 0.25) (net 10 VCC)))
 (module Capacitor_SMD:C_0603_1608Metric (layer F.Cu) (at 138.36 80.24)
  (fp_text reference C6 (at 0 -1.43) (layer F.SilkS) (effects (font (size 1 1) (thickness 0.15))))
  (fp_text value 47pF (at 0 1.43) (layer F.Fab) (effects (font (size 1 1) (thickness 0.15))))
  (pad 2 smd roundrect (at 0.775 0) (size 0.9 0.95) (layers F.Cu F.Paste F.Mask) (roundrect_rratio 0.25) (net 4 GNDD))
  (pad 1 smd roundrect (at -0.775 0) (size 0.9 0.95) (layers F.Cu F.Paste F.Mask) (roundrect_rratio 0.25) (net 27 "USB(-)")))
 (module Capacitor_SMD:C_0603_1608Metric (layer F.Cu) (at 114.3 93.95)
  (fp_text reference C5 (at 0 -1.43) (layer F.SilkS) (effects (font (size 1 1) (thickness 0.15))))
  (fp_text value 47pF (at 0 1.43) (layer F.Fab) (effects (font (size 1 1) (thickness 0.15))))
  (pad 2 smd roundrect (at 0.775 0) (size 0.9 0.95) (layers F.Cu F.Paste F.Mask) (roundrect_rratio 0.25) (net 4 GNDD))
  (pad 1 smd roundrect (at -0.775 0) (size 0.9 0.95) (layers F.Cu F.Paste F.Mask) (roundrect_rratio 0.25) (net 28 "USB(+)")))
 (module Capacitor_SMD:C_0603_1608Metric (layer F.Cu) (at 114.3 91.44)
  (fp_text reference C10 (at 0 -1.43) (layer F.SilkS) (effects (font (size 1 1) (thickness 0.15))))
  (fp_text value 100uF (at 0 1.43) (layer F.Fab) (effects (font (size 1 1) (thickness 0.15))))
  (pad 2 smd roundrect (at 0.775 0) (size 0.9 0.95) (layers F.Cu F.Paste F.Mask) (roundrect_rratio 0.25) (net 4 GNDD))
  (pad 1 smd roundrect (at -0.775 0) (size 0.9 0.95) (layers F.Cu F.Paste F.Mask) (roundrect_rratio 0.25) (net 14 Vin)))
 (gr_line (start 50.8 93.98) (end 50.8 76.2) (layer Edge.Cuts) (width 0.05))
 (gr_line (start 101.6 93.98) (end 50.8 93.98) (layer Edge.Cuts) (width 0.05))
 (gr_line (start 101.6 76.2) (end 101.6 93.98) (layer Edge.Cuts) (width 0.05))
 (gr_line (start 50.8 76.2) (end 101.6 76.2) (layer Edge.Cuts) (width 0.05))
 (segment (start 97.155 79.375) (end 95.25 77.47) (width 0.25) (layer F.Cu) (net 8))
 (segment (start 97.155 82.755002) (end 97.155 79.375) (width 0.25) (layer F.Cu) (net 8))
 (segment (start 98.219998 83.82) (end 97.155 82.755002) (width 0.25) (layer F.Cu) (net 8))
 (segment (start 99.105 83.82) (end 98.219998 83.82) (width 0.25) (layer F.Cu) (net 8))
 (segment (start 100.555 82.55) (end 100.965 82.14) (width 0.25) (layer F.Cu) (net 9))
 (segment (start 99.105 82.55) (end 100.555 82.55) (width 0.25) (layer F.Cu) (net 9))
 (segment (start 100.965 80.984998) (end 97.79 77.809998) (width 0.25) (layer F.Cu) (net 9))
 (segment (start 97.79 77.809998) (end 97.79 77.47) (width 0.25) (layer F.Cu) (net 9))
 (segment (start 100.965 82.14) (end 100.965 80.984998) (width 0.25) (layer F.Cu) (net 9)))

